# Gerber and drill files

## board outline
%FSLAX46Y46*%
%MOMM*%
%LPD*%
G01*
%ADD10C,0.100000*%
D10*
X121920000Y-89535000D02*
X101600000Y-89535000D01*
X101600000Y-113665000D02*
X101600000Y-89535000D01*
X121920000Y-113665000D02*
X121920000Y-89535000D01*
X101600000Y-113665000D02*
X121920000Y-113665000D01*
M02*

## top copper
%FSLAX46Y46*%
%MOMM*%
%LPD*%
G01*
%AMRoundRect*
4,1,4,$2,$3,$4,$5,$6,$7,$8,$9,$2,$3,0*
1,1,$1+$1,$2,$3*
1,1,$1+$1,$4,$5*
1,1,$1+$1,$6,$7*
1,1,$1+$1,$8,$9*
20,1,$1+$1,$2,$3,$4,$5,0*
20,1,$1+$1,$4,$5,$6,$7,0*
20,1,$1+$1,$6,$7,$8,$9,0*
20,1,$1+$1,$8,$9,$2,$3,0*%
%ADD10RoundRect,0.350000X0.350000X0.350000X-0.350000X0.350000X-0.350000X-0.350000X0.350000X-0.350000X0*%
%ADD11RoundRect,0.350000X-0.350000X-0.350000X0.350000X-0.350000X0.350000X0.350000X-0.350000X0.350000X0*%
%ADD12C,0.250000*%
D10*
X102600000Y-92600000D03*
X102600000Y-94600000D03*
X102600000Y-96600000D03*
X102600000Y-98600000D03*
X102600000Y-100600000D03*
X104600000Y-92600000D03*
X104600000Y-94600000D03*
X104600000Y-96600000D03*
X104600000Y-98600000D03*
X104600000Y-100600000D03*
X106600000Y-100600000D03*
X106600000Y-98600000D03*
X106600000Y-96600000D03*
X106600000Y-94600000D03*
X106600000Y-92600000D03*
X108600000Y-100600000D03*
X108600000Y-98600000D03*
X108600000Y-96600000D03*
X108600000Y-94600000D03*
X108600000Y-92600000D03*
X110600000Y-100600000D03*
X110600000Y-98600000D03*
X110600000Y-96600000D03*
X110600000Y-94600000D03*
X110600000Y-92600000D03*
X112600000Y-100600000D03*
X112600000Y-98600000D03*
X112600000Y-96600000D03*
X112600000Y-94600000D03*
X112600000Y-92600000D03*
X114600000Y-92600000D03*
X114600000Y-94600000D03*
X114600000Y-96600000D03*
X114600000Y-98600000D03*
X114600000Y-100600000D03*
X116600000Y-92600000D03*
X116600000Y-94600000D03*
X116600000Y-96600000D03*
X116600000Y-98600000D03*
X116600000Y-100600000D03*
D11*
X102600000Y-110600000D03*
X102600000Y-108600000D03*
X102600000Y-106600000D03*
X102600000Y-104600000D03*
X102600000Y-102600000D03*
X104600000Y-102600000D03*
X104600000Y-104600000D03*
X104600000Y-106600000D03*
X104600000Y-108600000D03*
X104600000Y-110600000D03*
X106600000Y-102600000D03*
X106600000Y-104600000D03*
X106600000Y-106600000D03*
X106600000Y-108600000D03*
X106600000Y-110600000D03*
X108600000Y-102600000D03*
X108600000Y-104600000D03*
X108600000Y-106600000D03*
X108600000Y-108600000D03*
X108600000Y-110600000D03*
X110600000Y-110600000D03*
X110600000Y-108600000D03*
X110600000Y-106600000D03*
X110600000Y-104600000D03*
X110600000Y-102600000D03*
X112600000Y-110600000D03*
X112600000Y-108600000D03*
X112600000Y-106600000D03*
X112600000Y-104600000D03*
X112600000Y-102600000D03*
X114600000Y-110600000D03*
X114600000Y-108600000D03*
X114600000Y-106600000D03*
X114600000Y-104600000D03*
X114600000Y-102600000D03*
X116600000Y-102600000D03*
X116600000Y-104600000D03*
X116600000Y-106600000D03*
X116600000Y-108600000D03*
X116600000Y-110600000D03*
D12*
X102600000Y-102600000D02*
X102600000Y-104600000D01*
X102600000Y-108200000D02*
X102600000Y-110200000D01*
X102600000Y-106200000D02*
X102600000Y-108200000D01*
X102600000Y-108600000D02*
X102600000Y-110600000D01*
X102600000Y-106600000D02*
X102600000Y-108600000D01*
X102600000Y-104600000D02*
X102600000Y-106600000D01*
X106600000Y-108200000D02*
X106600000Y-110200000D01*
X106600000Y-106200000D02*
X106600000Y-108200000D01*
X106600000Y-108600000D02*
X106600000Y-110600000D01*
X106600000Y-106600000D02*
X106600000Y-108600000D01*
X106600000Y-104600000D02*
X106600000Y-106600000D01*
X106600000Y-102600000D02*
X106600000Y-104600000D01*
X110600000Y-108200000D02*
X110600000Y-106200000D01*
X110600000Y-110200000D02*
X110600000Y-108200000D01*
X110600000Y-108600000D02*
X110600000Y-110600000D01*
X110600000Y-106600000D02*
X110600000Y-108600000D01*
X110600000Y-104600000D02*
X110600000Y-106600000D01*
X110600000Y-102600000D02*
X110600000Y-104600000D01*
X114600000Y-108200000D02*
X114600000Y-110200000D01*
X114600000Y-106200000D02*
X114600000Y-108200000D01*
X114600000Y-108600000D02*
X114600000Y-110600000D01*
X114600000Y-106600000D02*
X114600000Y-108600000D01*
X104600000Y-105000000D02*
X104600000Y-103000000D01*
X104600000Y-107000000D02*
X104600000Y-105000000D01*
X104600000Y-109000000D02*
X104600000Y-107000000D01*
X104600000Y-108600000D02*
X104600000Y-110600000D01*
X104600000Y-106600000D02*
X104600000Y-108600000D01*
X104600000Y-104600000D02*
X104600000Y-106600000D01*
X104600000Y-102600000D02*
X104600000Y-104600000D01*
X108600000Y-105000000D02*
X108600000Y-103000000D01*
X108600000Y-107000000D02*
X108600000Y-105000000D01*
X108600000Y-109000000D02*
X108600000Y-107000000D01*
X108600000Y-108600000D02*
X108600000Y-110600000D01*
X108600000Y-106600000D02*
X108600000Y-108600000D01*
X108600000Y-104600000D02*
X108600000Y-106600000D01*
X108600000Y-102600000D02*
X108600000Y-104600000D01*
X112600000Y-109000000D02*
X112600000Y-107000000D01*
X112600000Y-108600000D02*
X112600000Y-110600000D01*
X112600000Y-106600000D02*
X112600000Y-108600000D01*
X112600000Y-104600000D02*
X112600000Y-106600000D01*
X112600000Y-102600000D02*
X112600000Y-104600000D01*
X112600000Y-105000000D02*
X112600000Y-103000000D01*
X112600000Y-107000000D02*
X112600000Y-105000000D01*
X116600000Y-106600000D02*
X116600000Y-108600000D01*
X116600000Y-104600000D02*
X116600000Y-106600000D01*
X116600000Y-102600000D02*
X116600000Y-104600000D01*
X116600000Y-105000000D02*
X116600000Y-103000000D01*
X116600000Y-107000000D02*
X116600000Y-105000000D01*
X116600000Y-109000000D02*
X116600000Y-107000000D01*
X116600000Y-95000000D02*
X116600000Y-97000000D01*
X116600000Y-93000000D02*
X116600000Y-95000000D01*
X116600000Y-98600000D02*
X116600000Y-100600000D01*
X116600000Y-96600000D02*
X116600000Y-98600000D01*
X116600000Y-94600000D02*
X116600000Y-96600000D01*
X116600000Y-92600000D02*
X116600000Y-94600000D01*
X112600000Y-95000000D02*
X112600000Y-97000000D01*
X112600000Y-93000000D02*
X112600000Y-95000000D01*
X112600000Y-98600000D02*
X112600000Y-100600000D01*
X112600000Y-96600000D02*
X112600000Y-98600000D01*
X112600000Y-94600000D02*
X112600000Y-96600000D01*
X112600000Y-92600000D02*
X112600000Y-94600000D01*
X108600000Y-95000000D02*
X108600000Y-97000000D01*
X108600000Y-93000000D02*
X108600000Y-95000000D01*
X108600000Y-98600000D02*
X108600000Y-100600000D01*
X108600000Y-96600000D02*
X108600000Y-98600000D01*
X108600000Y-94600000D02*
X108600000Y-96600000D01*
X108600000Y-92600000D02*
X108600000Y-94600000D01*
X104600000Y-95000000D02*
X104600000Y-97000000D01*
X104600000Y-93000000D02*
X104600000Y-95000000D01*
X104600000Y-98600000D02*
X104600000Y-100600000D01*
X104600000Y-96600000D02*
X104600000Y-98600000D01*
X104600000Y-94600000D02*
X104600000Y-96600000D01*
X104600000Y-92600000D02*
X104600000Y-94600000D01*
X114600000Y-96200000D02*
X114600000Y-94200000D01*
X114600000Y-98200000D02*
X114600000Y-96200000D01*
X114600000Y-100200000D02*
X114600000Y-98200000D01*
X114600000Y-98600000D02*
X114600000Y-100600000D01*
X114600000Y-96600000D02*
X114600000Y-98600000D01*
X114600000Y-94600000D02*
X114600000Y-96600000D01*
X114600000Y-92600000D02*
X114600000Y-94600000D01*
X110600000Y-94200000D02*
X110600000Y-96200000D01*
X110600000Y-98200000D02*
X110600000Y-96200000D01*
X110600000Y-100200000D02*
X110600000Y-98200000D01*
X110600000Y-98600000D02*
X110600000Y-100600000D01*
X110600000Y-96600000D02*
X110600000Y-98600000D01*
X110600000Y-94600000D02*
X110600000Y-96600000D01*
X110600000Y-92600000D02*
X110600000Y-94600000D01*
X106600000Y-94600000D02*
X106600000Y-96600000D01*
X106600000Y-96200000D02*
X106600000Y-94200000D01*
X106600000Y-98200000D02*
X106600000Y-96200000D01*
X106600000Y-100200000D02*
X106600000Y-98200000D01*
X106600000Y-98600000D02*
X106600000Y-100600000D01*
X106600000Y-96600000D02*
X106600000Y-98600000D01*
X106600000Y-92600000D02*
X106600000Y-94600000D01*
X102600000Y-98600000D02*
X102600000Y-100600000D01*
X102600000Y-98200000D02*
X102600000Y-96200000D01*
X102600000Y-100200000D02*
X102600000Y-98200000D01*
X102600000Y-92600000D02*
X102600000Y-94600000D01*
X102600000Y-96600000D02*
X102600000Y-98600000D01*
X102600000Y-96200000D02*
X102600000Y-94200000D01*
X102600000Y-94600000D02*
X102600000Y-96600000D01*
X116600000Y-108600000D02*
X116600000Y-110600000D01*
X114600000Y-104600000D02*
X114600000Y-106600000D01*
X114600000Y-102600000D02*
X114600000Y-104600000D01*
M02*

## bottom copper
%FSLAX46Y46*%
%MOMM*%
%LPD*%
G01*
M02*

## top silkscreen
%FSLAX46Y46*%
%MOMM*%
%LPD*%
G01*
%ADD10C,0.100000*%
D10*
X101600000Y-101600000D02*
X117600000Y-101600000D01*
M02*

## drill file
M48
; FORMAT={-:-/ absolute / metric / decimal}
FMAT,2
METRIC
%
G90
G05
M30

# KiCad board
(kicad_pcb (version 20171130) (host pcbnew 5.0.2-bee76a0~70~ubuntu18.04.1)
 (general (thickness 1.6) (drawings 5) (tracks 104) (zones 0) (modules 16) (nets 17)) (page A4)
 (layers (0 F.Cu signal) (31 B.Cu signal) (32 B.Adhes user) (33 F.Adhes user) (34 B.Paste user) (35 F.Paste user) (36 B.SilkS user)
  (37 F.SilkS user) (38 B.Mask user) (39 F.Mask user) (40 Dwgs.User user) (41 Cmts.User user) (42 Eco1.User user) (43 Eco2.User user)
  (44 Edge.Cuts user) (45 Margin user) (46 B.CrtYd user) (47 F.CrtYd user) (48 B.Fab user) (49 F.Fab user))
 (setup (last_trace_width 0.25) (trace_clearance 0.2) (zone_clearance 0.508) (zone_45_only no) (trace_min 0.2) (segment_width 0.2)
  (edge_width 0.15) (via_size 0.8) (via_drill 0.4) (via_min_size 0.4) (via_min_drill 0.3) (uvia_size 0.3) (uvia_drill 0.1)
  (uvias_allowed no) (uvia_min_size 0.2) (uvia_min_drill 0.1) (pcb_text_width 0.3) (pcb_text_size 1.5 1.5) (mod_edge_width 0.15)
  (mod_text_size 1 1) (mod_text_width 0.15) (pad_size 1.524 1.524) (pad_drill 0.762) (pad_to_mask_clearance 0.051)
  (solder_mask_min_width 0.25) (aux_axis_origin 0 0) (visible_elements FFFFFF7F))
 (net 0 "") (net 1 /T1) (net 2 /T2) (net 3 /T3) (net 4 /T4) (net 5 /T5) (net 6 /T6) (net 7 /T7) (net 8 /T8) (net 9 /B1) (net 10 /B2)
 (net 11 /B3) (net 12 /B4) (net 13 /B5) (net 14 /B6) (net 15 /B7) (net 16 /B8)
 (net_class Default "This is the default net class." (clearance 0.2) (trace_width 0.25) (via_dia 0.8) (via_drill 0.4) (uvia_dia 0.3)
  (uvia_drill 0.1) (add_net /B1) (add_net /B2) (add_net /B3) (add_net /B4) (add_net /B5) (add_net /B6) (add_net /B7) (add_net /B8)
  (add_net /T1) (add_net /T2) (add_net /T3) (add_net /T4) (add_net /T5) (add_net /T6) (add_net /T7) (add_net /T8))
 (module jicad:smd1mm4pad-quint (layer F.Cu) (at 102.6 100.6 180)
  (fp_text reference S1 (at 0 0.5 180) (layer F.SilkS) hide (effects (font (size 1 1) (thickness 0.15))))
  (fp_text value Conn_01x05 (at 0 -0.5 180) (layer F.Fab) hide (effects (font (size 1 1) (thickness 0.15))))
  (pad 5 smd roundrect (at 0 8 180) (size 1.4 1.4) (layers F.Cu F.Paste F.Mask) (roundrect_rratio 0.25) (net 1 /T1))
  (pad 4 smd roundrect (at 0 6 180) (size 1.4 1.4) (layers F.Cu F.Paste F.Mask) (roundrect_rratio 0.25) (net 1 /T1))
  (pad 3 smd roundrect (at 0 4 180) (size 1.4 1.4) (layers F.Cu F.Paste F.Mask) (roundrect_rratio 0.25) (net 1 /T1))
  (pad 2 smd roundrect (at 0 2 180) (size 1.4 1.4) (layers F.Cu F.Paste F.Mask) (roundrect_rratio 0.25) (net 1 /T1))
  (pad 1 smd roundrect (at 0 0 180) (size 1.4 1.4) (layers F.Cu F.Paste F.Mask) (roundrect_rratio 0.25) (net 1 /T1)))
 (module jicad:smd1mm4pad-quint (layer F.Cu) (at 104.6 100.6 180)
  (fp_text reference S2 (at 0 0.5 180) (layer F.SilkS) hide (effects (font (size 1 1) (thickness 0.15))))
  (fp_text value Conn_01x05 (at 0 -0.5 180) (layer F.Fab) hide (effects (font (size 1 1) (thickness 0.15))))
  (pad 5 smd roundrect (at 0 8 180) (size 1.4 1.4) (layers F.Cu F.Paste F.Mask) (roundrect_rratio 0.25) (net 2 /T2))
  (pad 4 smd roundrect (at 0 6 180) (size 1.4 1.4) (layers F.Cu F.Paste F.Mask) (roundrect_rratio 0.25) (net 2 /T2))
  (pad 3 smd roundrect (at 0 4 180) (size 1.4 1.4) (layers F.Cu F.Paste F.Mask) (roundrect_rratio 0.25) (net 2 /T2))
  (pad 2 smd roundrect (at 0 2 180) (size 1.4 1.4) (layers F.Cu F.Paste F.Mask) (roundrect_rratio 0.25) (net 2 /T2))
  (pad 1 smd roundrect (at 0 0 180) (size 1.4 1.4) (layers F.Cu F.Paste F.Mask) (roundrect_rratio 0.25) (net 2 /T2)))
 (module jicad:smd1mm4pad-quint (layer F.Cu) (at 106.6 100.6 180)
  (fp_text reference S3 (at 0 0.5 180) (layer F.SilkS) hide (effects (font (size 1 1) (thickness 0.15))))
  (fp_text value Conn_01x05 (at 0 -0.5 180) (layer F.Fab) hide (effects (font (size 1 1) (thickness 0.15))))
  (pad 1 smd roundrect (at 0 0 180) (size 1.4 1.4) (layers F.Cu F.Paste F.Mask) (roundrect_rratio 0.25) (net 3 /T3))
  (pad 2 smd roundrect (at 0 2 180) (size 1.4 1.4) (layers F.Cu F.Paste F.Mask) (roundrect_rratio 0.25) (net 3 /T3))
  (pad 3 smd roundrect (at 0 4 180) (size 1.4 1.4) (layers F.Cu F.Paste F.Mask) (roundrect_rratio 0.25) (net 3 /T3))
  (pad 4 smd roundrect (at 0 6 180) (size 1.4 1.4) (layers F.Cu F.Paste F.Mask) (roundrect_rratio 0.25) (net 3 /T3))
  (pad 5 smd roundrect (at 0 8 180) (size 1.4 1.4) (layers F.Cu F.Paste F.Mask) (roundrect_rratio 0.25) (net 3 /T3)))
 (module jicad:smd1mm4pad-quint (layer F.Cu) (at 108.6 100.6 180)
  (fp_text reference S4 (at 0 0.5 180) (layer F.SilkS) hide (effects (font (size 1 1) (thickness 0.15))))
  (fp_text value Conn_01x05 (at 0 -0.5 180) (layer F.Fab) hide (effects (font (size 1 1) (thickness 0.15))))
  (pad 1 smd roundrect (at 0 0 180) (size 1.4 1.4) (layers F.Cu F.Paste F.Mask) (roundrect_rratio 0.25) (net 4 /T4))
  (pad 2 smd roundrect (at 0 2 180) (size 1.4 1.4) (layers F.Cu F.Paste F.Mask) (roundrect_rratio 0.25) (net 4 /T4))
  (pad 3 smd roundrect (at 0 4 180) (size 1.4 1.4) (layers F.Cu F.Paste F.Mask) (roundrect_rratio 0.25) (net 4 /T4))
  (pad 4 smd roundrect (at 0 6 180) (size 1.4 1.4) (layers F.Cu F.Paste F.Mask) (roundrect_rratio 0.25) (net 4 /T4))
  (pad 5 smd roundrect (at 0 8 180) (size 1.4 1.4) (layers F.Cu F.Paste F.Mask) (roundrect_rratio 0.25) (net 4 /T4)))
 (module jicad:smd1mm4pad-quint (layer F.Cu) (at 110.6 100.6 180)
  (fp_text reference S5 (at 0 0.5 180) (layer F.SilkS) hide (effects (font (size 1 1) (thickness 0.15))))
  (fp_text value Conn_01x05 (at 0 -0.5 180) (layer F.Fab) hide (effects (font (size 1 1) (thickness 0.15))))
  (pad 1 smd roundrect (at 0 0 180) (size 1.4 1.4) (layers F.Cu F.Paste F.Mask) (roundrect_rratio 0.25) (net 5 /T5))
  (pad 2 smd roundrect (at 0 2 180) (size 1.4 1.4) (layers F.Cu F.Paste F.Mask) (roundrect_rratio 0.25) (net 5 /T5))
  (pad 3 smd roundrect (at 0 4 180) (size 1.4 1.4) (layers F.Cu F.Paste F.Mask) (roundrect_rratio 0.25) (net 5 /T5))
  (pad 4 smd roundrect (at 0 6 180) (size 1.4 1.4) (layers F.Cu F.Paste F.Mask) (roundrect_rratio 0.25) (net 5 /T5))
  (pad 5 smd roundrect (at 0 8 180) (size 1.4 1.4) (layers F.Cu F.Paste F.Mask) (roundrect_rratio 0.25) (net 5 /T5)))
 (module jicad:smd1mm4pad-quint (layer F.Cu) (at 112.6 100.6 180)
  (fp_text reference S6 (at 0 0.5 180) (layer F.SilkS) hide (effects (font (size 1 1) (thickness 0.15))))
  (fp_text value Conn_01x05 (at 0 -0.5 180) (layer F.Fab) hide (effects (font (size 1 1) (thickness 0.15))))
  (pad 1 smd roundrect (at 0 0 180) (size 1.4 1.4) (layers F.Cu F.Paste F.Mask) (roundrect_rratio 0.25) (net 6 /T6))
  (pad 2 smd roundrect (at 0 2 180) (size 1.4 1.4) (layers F.Cu F.Paste F.Mask) (roundrect_rratio 0.25) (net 6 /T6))
  (pad 3 smd roundrect (at 0 4 180) (size 1.4 1.4) (layers F.Cu F.Paste F.Mask) (roundrect_rratio 0.25) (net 6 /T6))
  (pad 4 smd roundrect (at 0 6 180) (size 1.4 1.4) (layers F.Cu F.Paste F.Mask) (roundrect_rratio 0.25) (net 6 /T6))
  (pad 5 smd roundrect (at 0 8 180) (size 1.4 1.4) (layers F.Cu F.Paste F.Mask) (roundrect_rratio 0.25) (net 6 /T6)))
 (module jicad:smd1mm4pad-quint (layer F.Cu) (at 114.6 100.6 180)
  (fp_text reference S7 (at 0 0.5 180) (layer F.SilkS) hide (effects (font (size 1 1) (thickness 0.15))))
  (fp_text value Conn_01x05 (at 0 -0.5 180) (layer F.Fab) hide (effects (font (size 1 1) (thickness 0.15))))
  (pad 5 smd roundrect (at 0 8 180) (size 1.4 1.4) (layers F.Cu F.Paste F.Mask) (roundrect_rratio 0.25) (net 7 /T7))
  (pad 4 smd roundrect (at 0 6 180) (size 1.4 1.4) (layers F.Cu F.Paste F.Mask) (roundrect_rratio 0.25) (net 7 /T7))
  (pad 3 smd roundrect (at 0 4 180) (size 1.4 1.4) (layers F.Cu F.Paste F.Mask) (roundrect_rratio 0.25) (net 7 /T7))
  (pad 2 smd roundrect (at 0 2 180) (size 1.4 1.4) (layers F.Cu F.Paste F.Mask) (roundrect_rratio 0.25) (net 7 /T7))
  (pad 1 smd roundrect (at 0 0 180) (size 1.4 1.4) (layers F.Cu F.Paste F.Mask) (roundrect_rratio 0.25) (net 7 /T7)))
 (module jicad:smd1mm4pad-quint (layer F.Cu) (at 116.6 100.6 180)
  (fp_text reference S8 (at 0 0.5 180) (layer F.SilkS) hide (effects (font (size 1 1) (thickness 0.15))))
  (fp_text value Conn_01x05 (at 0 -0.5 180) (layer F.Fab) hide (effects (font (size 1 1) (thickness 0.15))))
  (pad 5 smd roundrect (at 0 8 180) (size 1.4 1.4) (layers F.Cu F.Paste F.Mask) (roundrect_rratio 0.25) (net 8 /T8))
  (pad 4 smd roundrect (at 0 6 180) (size 1.4 1.4) (layers F.Cu F.Paste F.Mask) (roundrect_rratio 0.25) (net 8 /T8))
  (pad 3 smd roundrect (at 0 4 180) (size 1.4 1.4) (layers F.Cu F.Paste F.Mask) (roundrect_rratio 0.25) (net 8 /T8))
  (pad 2 smd roundrect (at 0 2 180) (size 1.4 1.4) (layers F.Cu F.Paste F.Mask) (roundrect_rratio 0.25) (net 8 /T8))
  (pad 1 smd roundrect (at 0 0 180) (size 1.4 1.4) (layers F.Cu F.Paste F.Mask) (roundrect_rratio 0.25) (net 8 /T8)))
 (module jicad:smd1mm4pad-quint (layer F.Cu) (at 102.6 102.6)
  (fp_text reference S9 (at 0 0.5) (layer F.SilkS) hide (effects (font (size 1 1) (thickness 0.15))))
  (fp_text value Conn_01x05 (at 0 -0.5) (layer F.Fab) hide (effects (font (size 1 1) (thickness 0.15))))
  (pad 5 smd roundrect (at 0 8) (size 1.4 1.4) (layers F.Cu F.Paste F.Mask) (roundrect_rratio 0.25) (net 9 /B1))
  (pad 4 smd roundrect (at 0 6) (size 1.4 1.4) (layers F.Cu F.Paste F.Mask) (roundrect_rratio 0.25) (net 9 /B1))
  (pad 3 smd roundrect (at 0 4) (size 1.4 1.4) (layers F.Cu F.Paste F.Mask) (roundrect_rratio 0.25) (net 9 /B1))
  (pad 2 smd roundrect (at 0 2) (size 1.4 1.4) (layers F.Cu F.Paste F.Mask) (roundrect_rratio 0.25) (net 9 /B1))
  (pad 1 smd roundrect (at 0 0) (size 1.4 1.4) (layers F.Cu F.Paste F.Mask) (roundrect_rratio 0.25) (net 9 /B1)))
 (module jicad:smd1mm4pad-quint (layer F.Cu) (at 104.6 102.6)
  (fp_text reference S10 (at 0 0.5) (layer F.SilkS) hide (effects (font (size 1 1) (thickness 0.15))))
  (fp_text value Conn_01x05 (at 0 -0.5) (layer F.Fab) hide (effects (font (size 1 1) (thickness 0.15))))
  (pad 1 smd roundrect (at 0 0) (size 1.4 1.4) (layers F.Cu F.Paste F.Mask) (roundrect_rratio 0.25) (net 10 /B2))
  (pad 2 smd roundrect (at 0 2) (size 1.4 1.4) (layers F.Cu F.Paste F.Mask) (roundrect_rratio 0.25) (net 10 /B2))
  (pad 3 smd roundrect (at 0 4) (size 1.4 1.4) (layers F.Cu F.Paste F.Mask) (roundrect_rratio 0.25) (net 10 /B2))
  (pad 4 smd roundrect (at 0 6) (size 1.4 1.4) (layers F.Cu F.Paste F.Mask) (roundrect_rratio 0.25) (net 10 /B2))
  (pad 5 smd roundrect (at 0 8) (size 1.4 1.4) (layers F.Cu F.Paste F.Mask) (roundrect_rratio 0.25) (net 10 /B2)))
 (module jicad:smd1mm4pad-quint (layer F.Cu) (at 106.6 102.6)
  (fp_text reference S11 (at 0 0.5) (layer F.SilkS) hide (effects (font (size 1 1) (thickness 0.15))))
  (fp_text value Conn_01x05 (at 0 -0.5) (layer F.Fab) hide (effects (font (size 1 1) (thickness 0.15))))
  (pad 1 smd roundrect (at 0 0) (size 1.4 1.4) (layers F.Cu F.Paste F.Mask) (roundrect_rratio 0.25) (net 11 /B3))
  (pad 2 smd roundrect (at 0 2) (size 1.4 1.4) (layers F.Cu F.Paste F.Mask) (roundrect_rratio 0.25) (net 11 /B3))
  (pad 3 smd roundrect (at 0 4) (size 1.4 1.4) (layers F.Cu F.Paste F.Mask) (roundrect_rratio 0.25) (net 11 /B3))
  (pad 4 smd roundrect (at 0 6) (size 1.4 1.4) (layers F.Cu F.Paste F.Mask) (roundrect_rratio 0.25) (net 11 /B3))
  (pad 5 smd roundrect (at 0 8) (size 1.4 1.4) (layers F.Cu F.Paste F.Mask) (roundrect_rratio 0.25) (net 11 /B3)))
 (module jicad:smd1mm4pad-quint (layer F.Cu) (at 108.6 102.6)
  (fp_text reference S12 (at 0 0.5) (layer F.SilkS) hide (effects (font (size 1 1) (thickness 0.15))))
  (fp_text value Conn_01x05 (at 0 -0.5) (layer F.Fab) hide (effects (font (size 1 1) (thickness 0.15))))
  (pad 1 smd roundrect (at 0 0) (size 1.4 1.4) (layers F.Cu F.Paste F.Mask) (roundrect_rratio 0.25) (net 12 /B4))
  (pad 2 smd roundrect (at 0 2) (size 1.4 1.4) (layers F.Cu F.Paste F.Mask) (roundrect_rratio 0.25) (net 12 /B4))
  (pad 3 smd roundrect (at 0 4) (size 1.4 1.4) (layers F.Cu F.Paste F.Mask) (roundrect_rratio 0.25) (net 12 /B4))
  (pad 4 smd roundrect (at 0 6) (size 1.4 1.4) (layers F.Cu F.Paste F.Mask) (roundrect_rratio 0.25) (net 12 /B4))
  (pad 5 smd roundrect (at 0 8) (size 1.4 1.4) (layers F.Cu F.Paste F.Mask) (roundrect_rratio 0.25) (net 12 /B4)))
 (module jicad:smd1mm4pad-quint (layer F.Cu) (at 110.6 102.6)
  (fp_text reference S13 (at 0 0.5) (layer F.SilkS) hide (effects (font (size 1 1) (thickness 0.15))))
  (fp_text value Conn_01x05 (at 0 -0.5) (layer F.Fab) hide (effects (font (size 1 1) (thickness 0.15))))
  (pad 5 smd roundrect (at 0 8) (size 1.4 1.4) (layers F.Cu F.Paste F.Mask) (roundrect_rratio 0.25) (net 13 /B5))
  (pad 4 smd roundrect (at 0 6) (size 1.4 1.4) (layers F.Cu F.Paste F.Mask) (roundrect_rratio 0.25) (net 13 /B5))
  (pad 3 smd roundrect (at 0 4) (size 1.4 1.4) (layers F.Cu F.Paste F.Mask) (roundrect_rratio 0.25) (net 13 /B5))
  (pad 2 smd roundrect (at 0 2) (size 1.4 1.4) (layers F.Cu F.Paste F.Mask) (roundrect_rratio 0.25) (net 13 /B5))
  (pad 1 smd roundrect (at 0 0) (size 1.4 1.4) (layers F.Cu F.Paste F.Mask) (roundrect_rratio 0.25) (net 13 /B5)))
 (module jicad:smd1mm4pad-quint (layer F.Cu) (at 112.6 102.6)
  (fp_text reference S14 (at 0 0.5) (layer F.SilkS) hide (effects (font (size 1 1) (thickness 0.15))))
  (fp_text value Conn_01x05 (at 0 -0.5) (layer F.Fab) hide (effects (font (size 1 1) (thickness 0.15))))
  (pad 5 smd roundrect (at 0 8) (size 1.4 1.4) (layers F.Cu F.Paste F.Mask) (roundrect_rratio 0.25) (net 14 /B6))
  (pad 4 smd roundrect (at 0 6) (size 1.4 1.4) (layers F.Cu F.Paste F.Mask) (roundrect_rratio 0.25) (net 14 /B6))
  (pad 3 smd roundrect (at 0 4) (size 1.4 1.4) (layers F.Cu F.Paste F.Mask) (roundrect_rratio 0.25) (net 14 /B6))
  (pad 2 smd roundrect (at 0 2) (size 1.4 1.4) (layers F.Cu F.Paste F.Mask) (roundrect_rratio 0.25) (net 14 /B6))
  (pad 1 smd roundrect (at 0 0) (size 1.4 1.4) (layers F.Cu F.Paste F.Mask) (roundrect_rratio 0.25) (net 14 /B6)))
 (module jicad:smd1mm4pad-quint (layer F.Cu) (at 114.6 102.6)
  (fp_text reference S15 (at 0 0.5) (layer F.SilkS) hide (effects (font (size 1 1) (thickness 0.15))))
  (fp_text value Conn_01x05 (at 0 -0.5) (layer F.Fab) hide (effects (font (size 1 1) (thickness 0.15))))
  (pad 5 smd roundrect (at 0 8) (size 1.4 1.4) (layers F.Cu F.Paste F.Mask) (roundrect_rratio 0.25) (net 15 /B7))
  (pad 4 smd roundrect (at 0 6) (size 1.4 1.4) (layers F.Cu F.Paste F.Mask) (roundrect_rratio 0.25) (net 15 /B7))
  (pad 3 smd roundrect (at 0 4) (size 1.4 1.4) (layers F.Cu F.Paste F.Mask) (roundrect_rratio 0.25) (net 15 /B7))
  (pad 2 smd roundrect (at 0 2) (size 1.4 1.4) (layers F.Cu F.Paste F.Mask) (roundrect_rratio 0.25) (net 15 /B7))
  (pad 1 smd roundrect (at 0 0) (size 1.4 1.4) (layers F.Cu F.Paste F.Mask) (roundrect_rratio 0.25) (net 15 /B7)))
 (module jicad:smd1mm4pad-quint (layer F.Cu) (at 116.6 102.6)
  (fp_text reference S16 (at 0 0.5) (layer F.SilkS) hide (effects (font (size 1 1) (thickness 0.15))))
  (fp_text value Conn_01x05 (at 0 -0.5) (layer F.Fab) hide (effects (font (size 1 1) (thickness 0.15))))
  (pad 1 smd roundrect (at 0 0) (size 1.4 1.4) (layers F.Cu F.Paste F.Mask) (roundrect_rratio 0.25) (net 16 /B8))
  (pad 2 smd roundrect (at 0 2) (size 1.4 1.4) (layers F.Cu F.Paste F.Mask) (roundrect_rratio 0.25) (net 16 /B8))
  (pad 3 smd roundrect (at 0 4) (size 1.4 1.4) (layers F.Cu F.Paste F.Mask) (roundrect_rratio 0.25) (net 16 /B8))
  (pad 4 smd roundrect (at 0 6) (size 1.4 1.4) (layers F.Cu F.Paste F.Mask) (roundrect_rratio 0.25) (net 16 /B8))
  (pad 5 smd roundrect (at 0 8) (size 1.4 1.4) (layers F.Cu F.Paste F.Mask) (roundrect_rratio 0.25) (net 16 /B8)))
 (gr_line (start 101.6 101.6) (end 117.6 101.6) (layer F.SilkS) (width 0.1))
 (gr_line (start 121.92 89.535) (end 101.6 89.535) (layer Edge.Cuts) (width 0.1))
 (gr_line (start 101.6 113.665) (end 101.6 89.535) (layer Edge.Cuts) (width 0.1))
 (gr_line (start 121.92 113.665) (end 121.92 89.535) (layer Edge.Cuts) (width 0.1))
 (gr_line (start 101.6 113.665) (end 121.92 113.665) (layer Edge.Cuts) (width 0.1))
 (segment (start 102.6 102.6) (end 102.6 104.6) (width 0.25) (layer F.Cu) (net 9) (status 30))
 (segment (start 102.6 108.2) (end 102.6 110.2) (width 0.25) (layer F.Cu) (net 9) (status 30))
 (segment (start 102.6 106.2) (end 102.6 108.2) (width 0.25) (layer F.Cu) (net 9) (status 30))
 (segment (start 102.6 108.6) (end 102.6 110.6) (width 0.25) (layer F.Cu) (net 9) (status 30))
 (segment (start 102.6 106.6) (end 102.6 108.6) (width 0.25) (layer F.Cu) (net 9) (status 30))
 (segment (start 102.6 104.6) (end 102.6 106.6) (width 0.25) (layer F.Cu) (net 9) (status 30))
 (segment (start 106.6 108.2) (end 106.6 110.2) (width 0.25) (layer F.Cu) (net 11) (status 30))
 (segment (start 106.6 106.2) (end 106.6 108.2) (width 0.25) (layer F.Cu) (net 11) (status 30))
 (segment (start 106.6 108.6) (end 106.6 110.6) (width 0.25) (layer F.Cu) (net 11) (status 30))
 (segment (start 106.6 106.6) (end 106.6 108.6) (width 0.25) (layer F.Cu) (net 11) (status 30))
 (segment (start 106.6 104.6) (end 106.6 106.6) (width 0.25) (layer F.Cu) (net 11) (status 30))
 (segment (start 106.6 102.6) (end 106.6 104.6) (width 0.25) (layer F.Cu) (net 11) (status 30))
 (segment (start 110.6 108.2) (end 110.6 106.2) (width 0.25) (layer F.Cu) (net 13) (status 30))
 (segment (start 110.6 110.2) (end 110.6 108.2) (width 0.25) (layer F.Cu) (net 13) (status 30))
 (segment (start 110.6 108.6) (end 110.6 110.6) (width 0.25) (layer F.Cu) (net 13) (status 30))
 (segment (start 110.6 106.6) (end 110.6 108.6) (width 0.25) (layer F.Cu) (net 13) (status 30))
 (segment (start 110.6 104.6) (end 110.6 106.6) (width 0.25) (layer F.Cu) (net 13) (status 30))
 (segment (start 110.6 102.6) (end 110.6 104.6) (width 0.25) (layer F.Cu) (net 13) (status 30))
 (segment (start 114.6 108.2) (end 114.6 110.2) (width 0.25) (layer F.Cu) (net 15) (status 30))
 (segment (start 114.6 106.2) (end 114.6 108.2) (width 0.25) (layer F.Cu) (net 15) (status 30))
 (segment (start 114.6 108.6) (end 114.6 110.6) (width 0.25) (layer F.Cu) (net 15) (status 30))
 (segment (start 114.6 106.6) (end 114.6 108.6) (width 0.25) (layer F.Cu) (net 15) (status 30))
 (segment (start 104.6 105) (end 104.6 103) (width 0.25) (layer F.Cu) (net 10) (status 30))
 (segment (start 104.6 107) (end 104.6 105) (width 0.25) (layer F.Cu) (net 10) (status 30))
 (segment (start 104.6 109) (end 104.6 107) (width 0.25) (layer F.Cu) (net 10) (status 30))
 (segment (start 104.6 108.6) (end 104.6 110.6) (width 0.25) (layer F.Cu) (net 10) (status 30))
 (segment (start 104.6 106.6) (end 104.6 108.6) (width 0.25) (layer F.Cu) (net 10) (status 30))
 (segment (start 104.6 104.6) (end 104.6 106.6) (width 0.25) (layer F.Cu) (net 10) (status 30))
 (segment (start 104.6 102.6) (end 104.6 104.6) (width 0.25) (layer F.Cu) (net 10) (status 30))
 (segment (start 108.6 105) (end 108.6 103) (width 0.25) (layer F.Cu) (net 12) (status 30))
 (segment (start 108.6 107) (end 108.6 105) (width 0.25) (layer F.Cu) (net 12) (status 30))
 (segment (start 108.6 109) (end 108.6 107) (width 0.25) (layer F.Cu) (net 12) (status 30))
 (segment (start 108.6 108.6) (end 108.6 110.6) (width 0.25) (layer F.Cu) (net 12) (status 30))
 (segment (start 108.6 106.6) (end 108.6 108.6) (width 0.25) (layer F.Cu) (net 12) (status 30))
 (segment (start 108.6 104.6) (end 108.6 106.6) (width 0.25) (layer F.Cu) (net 12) (status 30))
 (segment (start 108.6 102.6) (end 108.6 104.6) (width 0.25) (layer F.Cu) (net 12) (status 30))
 (segment (start 112.6 109) (end 112.6 107) (width 0.25) (layer F.Cu) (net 14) (status 30))
 (segment (start 112.6 108.6) (end 112.6 110.6) (width 0.25) (layer F.Cu) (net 14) (status 30))
 (segment (start 112.6 106.6) (end 112.6 108.6) (width 0.25) (layer F.Cu) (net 14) (status 30))
 (segment (start 112.6 104.6) (end 112.6 106.6) (width 0.25) (layer F.Cu) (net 14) (status 30))
 (segment (start 112.6 102.6) (end 112.6 104.6) (width 0.25) (layer F.Cu) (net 14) (status 30))
 (segment (start 112.6 105) (end 112.6 103) (width 0.25) (layer F.Cu) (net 14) (status 30))
 (segment (start 112.6 107) (end 112.6 105) (width 0.25) (layer F.Cu) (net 14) (status 30))
 (segment (start 116.6 106.6) (end 116.6 108.6) (width 0.25) (layer F.Cu) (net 16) (status 30))
 (segment (start 116.6 104.6) (end 116.6 106.6) (width 0.25) (layer F.Cu) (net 16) (status 30))
 (segment (start 116.6 102.6) (end 116.6 104.6) (width 0.25) (layer F.Cu) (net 16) (status 30))
 (segment (start 116.6 105) (end 116.6 103) (width 0.25) (layer F.Cu) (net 16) (status 30))
 (segment (start 116.6 107) (end 116.6 105) (width 0.25) (layer F.Cu) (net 16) (status 30))
 (segment (start 116.6 109) (end 116.6 107) (width 0.25) (layer F.Cu) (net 16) (status 30))
 (segment (start 116.6 95) (end 116.6 97) (width 0.25) (layer F.Cu) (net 8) (status 30))
 (segment (start 116.6 93) (end 116.6 95) (width 0.25) (layer F.Cu) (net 8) (status 30))
 (segment (start 116.6 98.6) (end 116.6 100.6) (width 0.25) (layer F.Cu) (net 8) (status 30))
 (segment (start 116.6 96.6) (end 116.6 98.6) (width 0.25) (layer F.Cu) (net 8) (status 30))
 (segment (start 116.6 94.6) (end 116.6 96.6) (width 0.25) (layer F.Cu) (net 8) (status 30))
 (segment (start 116.6 92.6) (end 116.6 94.6) (width 0.25) (layer F.Cu) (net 8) (status 30))
 (segment (start 112.6 95) (end 112.6 97) (width 0.25) (layer F.Cu) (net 6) (status 30))
 (segment (start 112.6 93) (end 112.6 95) (width 0.25) (layer F.Cu) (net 6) (status 30))
 (segment (start 112.6 98.6) (end 112.6 100.6) (width 0.25) (layer F.Cu) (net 6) (status 30))
 (segment (start 112.6 96.6) (end 112.6 98.6) (width 0.25) (layer F.Cu) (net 6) (status 30))
 (segment (start 112.6 94.6) (end 112.6 96.6) (width 0.25) (layer F.Cu) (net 6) (status 30))
 (segment (start 112.6 92.6) (end 112.6 94.6) (width 0.25) (layer F.Cu) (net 6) (status 30))
 (segment (start 108.6 95) (end 108.6 97) (width 0.25) (layer F.Cu) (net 4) (status 30))
 (segment (start 108.6 93) (end 108.6 95) (width 0.25) (layer F.Cu) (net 4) (status 30))
 (segment (start 108.6 98.6) (end 108.6 100.6) (width 0.25) (layer F.Cu) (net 4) (status 30))
 (segment (start 108.6 96.6) (end 108.6 98.6) (width 0.25) (layer F.Cu) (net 4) (status 30))
 (segment (start 108.6 94.6) (end 108.6 96.6) (width 0.25) (layer F.Cu) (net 4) (status 30))
 (segment (start 108.6 92.6) (end 108.6 94.6) (width 0.25) (layer F.Cu) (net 4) (status 30))
 (segment (start 104.6 95) (end 104.6 97) (width 0.25) (layer F.Cu) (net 2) (status 30))
 (segment (start 104.6 93) (end 104.6 95) (width 0.25) (layer F.Cu) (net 2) (status 30))
 (segment (start 104.6 98.6) (end 104.6 100.6) (width 0.25) (layer F.Cu) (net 2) (status 30))
 (segment (start 104.6 96.6) (end 104.6 98.6) (width 0.25) (layer F.Cu) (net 2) (status 30))
 (segment (start 104.6 94.6) (end 104.6 96.6) (width 0.25) (layer F.Cu) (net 2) (status 30))
 (segment (start 104.6 92.6) (end 104.6 94.6) (width 0.25) (layer F.Cu) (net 2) (status 30))
 (segment (start 114.6 96.2) (end 114.6 94.2) (width 0.25) (layer F.Cu) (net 7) (status 30))
 (segment (start 114.6 98.2) (end 114.6 96.2) (width 0.25) (layer F.Cu) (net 7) (status 30))
 (segment (start 114.6 100.2) (end 114.6 98.2) (width 0.25) (layer F.Cu) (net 7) (status 30))
 (segment (start 114.6 98.6) (end 114.6 100.6) (width 0.25) (layer F.Cu) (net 7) (status 30))
 (segment (start 114.6 96.6) (end 114.6 98.6) (width 0.25) (layer F.Cu) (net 7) (status 30))
 (segment (start 114.6 94.6) (end 114.6 96.6) (width 0.25) (layer F.Cu) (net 7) (status 30))
 (segment (start 114.6 92.6) (end 114.6 94.6) (width 0.25) (layer F.Cu) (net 7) (status 30))
 (segment (start 110.6 94.2) (end 110.6 96.2) (width 0.25) (layer F.Cu) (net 5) (status 30))
 (segment (start 110.6 98.2) (end 110.6 96.2) (width 0.25) (layer F.Cu) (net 5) (status 30))
 (segment (start 110.6 100.2) (end 110.6 98.2) (width 0.25) (layer F.Cu) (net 5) (status 30))
 (segment (start 110.6 98.6) (end 110.6 100.6) (width 0.25) (layer F.Cu) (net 5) (status 30))
 (segment (start 110.6 96.6) (end 110.6 98.6) (width 0.25) (layer F.Cu) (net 5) (status 30))
 (segment (start 110.6 94.6) (end 110.6 96.6) (width 0.25) (layer F.Cu) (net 5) (status 30))
 (segment (start 110.6 92.6) (end 110.6 94.6) (width 0.25) (layer F.Cu) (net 5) (status 30))
 (segment (start 106.6 94.6) (end 106.6 96.6) (width 0.25) (layer F.Cu) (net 3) (status 30))
 (segment (start 106.6 96.2) (end 106.6 94.2) (width 0.25) (layer F.Cu) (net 3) (status 30))
 (segment (start 106.6 98.2) (end 106.6 96.2) (width 0.25) (layer F.Cu) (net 3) (status 30))
 (segment (start 106.6 100.2) (end 106.6 98.2) (width 0.25) (layer F.Cu) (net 3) (status 30))
 (segment (start 106.6 98.6) (end 106.6 100.6) (width 0.25) (layer F.Cu) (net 3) (status 30))
 (segment (start 106.6 96.6) (end 106.6 98.6) (width 0.25) (layer F.Cu) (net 3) (status 30))
 (segment (start 106.6 92.6) (end 106.6 94.6) (width 0.25) (layer F.Cu) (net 3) (status 30))
 (segment (start 102.6 98.6) (end 102.6 100.6) (width 0.25) (layer F.Cu) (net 1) (status 30))
 (segment (start 102.6 98.2) (end 102.6 96.2) (width 0.25) (layer F.Cu) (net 1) (status 30))
 (segment (start 102.6 100.2) (end 102.6 98.2) (width 0.25) (layer F.Cu) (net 1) (status 30))
 (segment (start 102.6 92.6) (end 102.6 94.6) (width 0.25) (layer F.Cu) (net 1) (status 30))
 (segment (start 102.6 96.6) (end 102.6 98.6) (width 0.25) (layer F.Cu) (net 1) (status 30))
 (segment (start 102.6 96.2) (end 102.6 94.2) (width 0.25) (layer F.Cu) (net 1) (status 30))
 (segment (start 102.6 94.6) (end 102.6 96.6) (width 0.25) (layer F.Cu) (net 1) (status 30))
 (segment (start 116.6 108.6) (end 116.6 110.6) (width 0.25) (layer F.Cu) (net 16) (status 30))
 (segment (start 114.6 104.6) (end 114.6 106.6) (width 0.25) (layer F.Cu) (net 15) (status 30))
 (segment (start 114.6 102.6) (end 114.6 104.6) (width 0.25) (layer F.Cu) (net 15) (status 30)))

